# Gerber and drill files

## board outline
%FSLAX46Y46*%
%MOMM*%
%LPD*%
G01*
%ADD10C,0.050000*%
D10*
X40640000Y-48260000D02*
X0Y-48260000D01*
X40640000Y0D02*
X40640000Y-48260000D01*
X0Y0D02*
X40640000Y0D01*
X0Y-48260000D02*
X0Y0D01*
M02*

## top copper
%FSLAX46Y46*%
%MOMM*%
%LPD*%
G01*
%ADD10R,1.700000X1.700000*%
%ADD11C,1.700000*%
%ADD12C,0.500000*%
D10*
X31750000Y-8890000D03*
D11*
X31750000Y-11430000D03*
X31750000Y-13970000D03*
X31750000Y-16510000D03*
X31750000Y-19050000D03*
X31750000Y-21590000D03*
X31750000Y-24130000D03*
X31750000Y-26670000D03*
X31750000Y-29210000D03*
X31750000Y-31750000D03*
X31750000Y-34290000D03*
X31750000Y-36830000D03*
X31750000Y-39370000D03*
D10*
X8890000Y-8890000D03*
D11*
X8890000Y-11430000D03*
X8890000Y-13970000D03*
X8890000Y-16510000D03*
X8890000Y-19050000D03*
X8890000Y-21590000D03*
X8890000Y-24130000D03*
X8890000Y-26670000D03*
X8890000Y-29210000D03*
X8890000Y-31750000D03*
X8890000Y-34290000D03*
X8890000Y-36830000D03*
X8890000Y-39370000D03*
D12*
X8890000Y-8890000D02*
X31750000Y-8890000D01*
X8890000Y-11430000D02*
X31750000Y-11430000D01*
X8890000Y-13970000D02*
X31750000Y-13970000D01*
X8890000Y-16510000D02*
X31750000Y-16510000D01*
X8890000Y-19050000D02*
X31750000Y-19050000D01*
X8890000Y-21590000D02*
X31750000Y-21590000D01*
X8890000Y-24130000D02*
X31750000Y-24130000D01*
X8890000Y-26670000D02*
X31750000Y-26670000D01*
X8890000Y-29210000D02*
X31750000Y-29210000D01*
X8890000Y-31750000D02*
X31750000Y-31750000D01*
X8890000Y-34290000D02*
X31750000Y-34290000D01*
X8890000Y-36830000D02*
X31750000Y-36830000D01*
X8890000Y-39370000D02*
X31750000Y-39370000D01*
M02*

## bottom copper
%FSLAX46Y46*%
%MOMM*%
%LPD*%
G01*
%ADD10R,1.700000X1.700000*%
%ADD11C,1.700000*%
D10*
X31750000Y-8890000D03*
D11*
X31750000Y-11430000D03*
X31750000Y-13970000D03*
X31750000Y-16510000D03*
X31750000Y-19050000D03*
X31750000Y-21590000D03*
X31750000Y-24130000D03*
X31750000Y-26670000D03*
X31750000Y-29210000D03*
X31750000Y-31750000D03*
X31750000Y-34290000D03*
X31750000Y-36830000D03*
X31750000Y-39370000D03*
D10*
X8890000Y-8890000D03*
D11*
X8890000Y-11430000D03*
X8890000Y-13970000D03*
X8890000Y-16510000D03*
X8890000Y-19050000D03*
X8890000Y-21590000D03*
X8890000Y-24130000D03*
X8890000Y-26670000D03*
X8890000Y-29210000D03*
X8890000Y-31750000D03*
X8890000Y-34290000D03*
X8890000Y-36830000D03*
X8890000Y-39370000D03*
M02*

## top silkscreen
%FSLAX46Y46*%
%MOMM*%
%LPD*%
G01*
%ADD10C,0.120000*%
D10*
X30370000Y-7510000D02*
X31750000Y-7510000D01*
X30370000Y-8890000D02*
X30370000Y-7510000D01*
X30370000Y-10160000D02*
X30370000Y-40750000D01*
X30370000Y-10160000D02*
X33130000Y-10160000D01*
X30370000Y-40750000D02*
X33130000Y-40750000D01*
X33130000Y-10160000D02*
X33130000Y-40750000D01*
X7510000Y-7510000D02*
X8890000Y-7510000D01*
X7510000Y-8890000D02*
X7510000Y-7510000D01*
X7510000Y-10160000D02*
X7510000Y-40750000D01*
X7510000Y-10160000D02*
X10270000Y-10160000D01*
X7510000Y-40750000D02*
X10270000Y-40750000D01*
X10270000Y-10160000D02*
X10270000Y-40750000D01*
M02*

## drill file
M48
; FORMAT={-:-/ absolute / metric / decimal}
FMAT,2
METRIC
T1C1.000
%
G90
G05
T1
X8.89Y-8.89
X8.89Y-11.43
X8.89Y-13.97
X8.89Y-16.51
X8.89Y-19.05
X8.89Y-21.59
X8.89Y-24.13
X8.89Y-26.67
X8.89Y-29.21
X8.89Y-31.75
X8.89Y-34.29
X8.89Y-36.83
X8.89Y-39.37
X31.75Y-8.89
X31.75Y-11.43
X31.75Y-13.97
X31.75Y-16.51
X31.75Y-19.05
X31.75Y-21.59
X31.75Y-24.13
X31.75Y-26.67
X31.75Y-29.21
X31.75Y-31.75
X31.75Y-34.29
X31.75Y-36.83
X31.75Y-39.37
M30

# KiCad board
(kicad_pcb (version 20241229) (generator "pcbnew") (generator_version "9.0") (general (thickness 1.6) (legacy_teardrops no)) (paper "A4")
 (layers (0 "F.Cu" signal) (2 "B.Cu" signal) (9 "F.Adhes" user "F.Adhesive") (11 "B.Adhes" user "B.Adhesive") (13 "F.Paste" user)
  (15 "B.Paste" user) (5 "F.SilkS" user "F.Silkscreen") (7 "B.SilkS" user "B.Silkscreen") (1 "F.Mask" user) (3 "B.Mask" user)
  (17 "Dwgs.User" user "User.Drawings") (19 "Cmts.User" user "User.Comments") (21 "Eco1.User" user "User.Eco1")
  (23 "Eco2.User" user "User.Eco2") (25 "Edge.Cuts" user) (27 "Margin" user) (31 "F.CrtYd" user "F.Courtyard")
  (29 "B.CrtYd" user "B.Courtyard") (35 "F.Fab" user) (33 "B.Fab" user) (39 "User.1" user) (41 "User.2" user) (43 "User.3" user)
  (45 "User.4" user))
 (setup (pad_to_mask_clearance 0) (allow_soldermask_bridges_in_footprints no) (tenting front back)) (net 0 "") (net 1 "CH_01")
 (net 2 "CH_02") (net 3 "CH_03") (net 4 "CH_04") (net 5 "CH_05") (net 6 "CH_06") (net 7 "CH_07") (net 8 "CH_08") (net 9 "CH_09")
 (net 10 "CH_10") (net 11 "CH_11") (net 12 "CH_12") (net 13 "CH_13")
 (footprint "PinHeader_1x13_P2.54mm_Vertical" (layer "F.Cu") (at 31.75 8.89)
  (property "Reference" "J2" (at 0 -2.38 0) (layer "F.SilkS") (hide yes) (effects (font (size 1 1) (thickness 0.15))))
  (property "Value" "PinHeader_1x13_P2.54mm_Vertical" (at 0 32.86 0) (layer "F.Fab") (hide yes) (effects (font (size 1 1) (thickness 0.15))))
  (fp_line (start -1.38 -1.38) (end 0 -1.38) (stroke (width 0.12) (type solid)) (layer "F.SilkS"))
  (fp_line (start -1.38 0) (end -1.38 -1.38) (stroke (width 0.12) (type solid)) (layer "F.SilkS"))
  (fp_line (start -1.38 1.27) (end -1.38 31.86) (stroke (width 0.12) (type solid)) (layer "F.SilkS"))
  (fp_line (start -1.38 1.27) (end 1.38 1.27) (stroke (width 0.12) (type solid)) (layer "F.SilkS"))
  (fp_line (start -1.38 31.86) (end 1.38 31.86) (stroke (width 0.12) (type solid)) (layer "F.SilkS"))
  (fp_line (start 1.38 1.27) (end 1.38 31.86) (stroke (width 0.12) (type solid)) (layer "F.SilkS"))
  (pad "1" thru_hole rect (at 0 0) (size 1.7 1.7) (drill 1) (layers "*.Cu" "*.Mask") (remove_unused_layers no) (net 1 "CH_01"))
  (pad "2" thru_hole circle (at 0 2.54) (size 1.7 1.7) (drill 1) (layers "*.Cu" "*.Mask") (remove_unused_layers no) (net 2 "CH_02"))
  (pad "3" thru_hole circle (at 0 5.08) (size 1.7 1.7) (drill 1) (layers "*.Cu" "*.Mask") (remove_unused_layers no) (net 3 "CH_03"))
  (pad "4" thru_hole circle (at 0 7.62) (size 1.7 1.7) (drill 1) (layers "*.Cu" "*.Mask") (remove_unused_layers no) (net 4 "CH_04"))
  (pad "5" thru_hole circle (at 0 10.16) (size 1.7 1.7) (drill 1) (layers "*.Cu" "*.Mask") (remove_unused_layers no) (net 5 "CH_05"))
  (pad "6" thru_hole circle (at 0 12.7) (size 1.7 1.7) (drill 1) (layers "*.Cu" "*.Mask") (remove_unused_layers no) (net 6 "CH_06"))
  (pad "7" thru_hole circle (at 0 15.24) (size 1.7 1.7) (drill 1) (layers "*.Cu" "*.Mask") (remove_unused_layers no) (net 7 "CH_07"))
  (pad "8" thru_hole circle (at 0 17.78) (size 1.7 1.7) (drill 1) (layers "*.Cu" "*.Mask") (remove_unused_layers no) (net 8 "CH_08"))
  (pad "9" thru_hole circle (at 0 20.32) (size 1.7 1.7) (drill 1) (layers "*.Cu" "*.Mask") (remove_unused_layers no) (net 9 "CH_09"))
  (pad "10" thru_hole circle (at 0 22.86) (size 1.7 1.7) (drill 1) (layers "*.Cu" "*.Mask") (remove_unused_layers no) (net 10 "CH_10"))
  (pad "11" thru_hole circle (at 0 25.4) (size 1.7 1.7) (drill 1) (layers "*.Cu" "*.Mask") (remove_unused_layers no) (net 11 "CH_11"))
  (pad "12" thru_hole circle (at 0 27.94) (size 1.7 1.7) (drill 1) (layers "*.Cu" "*.Mask") (remove_unused_layers no) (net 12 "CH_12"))
  (pad "13" thru_hole circle (at 0 30.48) (size 1.7 1.7) (drill 1) (layers "*.Cu" "*.Mask") (remove_unused_layers no) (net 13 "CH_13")))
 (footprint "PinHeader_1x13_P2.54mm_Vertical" (layer "F.Cu") (at 8.89 8.89)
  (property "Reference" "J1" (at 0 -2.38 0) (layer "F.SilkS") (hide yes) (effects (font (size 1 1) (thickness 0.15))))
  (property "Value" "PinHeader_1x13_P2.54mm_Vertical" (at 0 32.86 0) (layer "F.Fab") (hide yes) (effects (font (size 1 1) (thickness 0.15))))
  (fp_line (start -1.38 -1.38) (end 0 -1.38) (stroke (width 0.12) (type solid)) (layer "F.SilkS"))
  (fp_line (start -1.38 0) (end -1.38 -1.38) (stroke (width 0.12) (type solid)) (layer "F.SilkS"))
  (fp_line (start -1.38 1.27) (end -1.38 31.86) (stroke (width 0.12) (type solid)) (layer "F.SilkS"))
  (fp_line (start -1.38 1.27) (end 1.38 1.27) (stroke (width 0.12) (type solid)) (layer "F.SilkS"))
  (fp_line (start -1.38 31.86) (end 1.38 31.86) (stroke (width 0.12) (type solid)) (layer "F.SilkS"))
  (fp_line (start 1.38 1.27) (end 1.38 31.86) (stroke (width 0.12) (type solid)) (layer "F.SilkS"))
  (pad "1" thru_hole rect (at 0 0) (size 1.7 1.7) (drill 1) (layers "*.Cu" "*.Mask") (remove_unused_layers no) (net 1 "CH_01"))
  (pad "2" thru_hole circle (at 0 2.54) (size 1.7 1.7) (drill 1) (layers "*.Cu" "*.Mask") (remove_unused_layers no) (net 2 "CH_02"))
  (pad "3" thru_hole circle (at 0 5.08) (size 1.7 1.7) (drill 1) (layers "*.Cu" "*.Mask") (remove_unused_layers no) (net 3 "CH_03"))
  (pad "4" thru_hole circle (at 0 7.62) (size 1.7 1.7) (drill 1) (layers "*.Cu" "*.Mask") (remove_unused_layers no) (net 4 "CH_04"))
  (pad "5" thru_hole circle (at 0 10.16) (size 1.7 1.7) (drill 1) (layers "*.Cu" "*.Mask") (remove_unused_layers no) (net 5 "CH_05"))
  (pad "6" thru_hole circle (at 0 12.7) (size 1.7 1.7) (drill 1) (layers "*.Cu" "*.Mask") (remove_unused_layers no) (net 6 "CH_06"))
  (pad "7" thru_hole circle (at 0 15.24) (size 1.7 1.7) (drill 1) (layers "*.Cu" "*.Mask") (remove_unused_layers no) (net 7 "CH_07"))
  (pad "8" thru_hole circle (at 0 17.78) (size 1.7 1.7) (drill 1) (layers "*.Cu" "*.Mask") (remove_unused_layers no) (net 8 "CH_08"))
  (pad "9" thru_hole circle (at 0 20.32) (size 1.7 1.7) (drill 1) (layers "*.Cu" "*.Mask") (remove_unused_layers no) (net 9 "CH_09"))
  (pad "10" thru_hole circle (at 0 22.86) (size 1.7 1.7) (drill 1) (layers "*.Cu" "*.Mask") (remove_unused_layers no) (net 10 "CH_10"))
  (pad "11" thru_hole circle (at 0 25.4) (size 1.7 1.7) (drill 1) (layers "*.Cu" "*.Mask") (remove_unused_layers no) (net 11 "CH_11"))
  (pad "12" thru_hole circle (at 0 27.94) (size 1.7 1.7) (drill 1) (layers "*.Cu" "*.Mask") (remove_unused_layers no) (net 12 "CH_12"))
  (pad "13" thru_hole circle (at 0 30.48) (size 1.7 1.7) (drill 1) (layers "*.Cu" "*.Mask") (remove_unused_layers no) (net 13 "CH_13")))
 (gr_line (start 40.64 48.26) (end 0 48.26) (stroke (width 0.05) (type default)) (layer "Edge.Cuts"))
 (gr_line (start 40.64 0) (end 40.64 48.26) (stroke (width 0.05) (type default)) (layer "Edge.Cuts"))
 (gr_line (start 0 0) (end 40.64 0) (stroke (width 0.05) (type default)) (layer "Edge.Cuts"))
 (gr_line (start 0 48.26) (end 0 0) (stroke (width 0.05) (type default)) (layer "Edge.Cuts"))
 (segment (start 8.89 8.89) (end 31.75 8.89) (width 0.5) (layer "F.Cu") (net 1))
 (segment (start 8.89 11.43) (end 31.75 11.43) (width 0.5) (layer "F.Cu") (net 2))
 (segment (start 8.89 13.97) (end 31.75 13.97) (width 0.5) (layer "F.Cu") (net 3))
 (segment (start 8.89 16.51) (end 31.75 16.51) (width 0.5) (layer "F.Cu") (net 4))
 (segment (start 8.89 19.05) (end 31.75 19.05) (width 0.5) (layer "F.Cu") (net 5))
 (segment (start 8.89 21.59) (end 31.75 21.59) (width 0.5) (layer "F.Cu") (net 6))
 (segment (start 8.89 24.13) (end 31.75 24.13) (width 0.5) (layer "F.Cu") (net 7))
 (segment (start 8.89 26.67) (end 31.75 26.67) (width 0.5) (layer "F.Cu") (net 8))
 (segment (start 8.89 29.21) (end 31.75 29.21) (width 0.5) (layer "F.Cu") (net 9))
 (segment (start 8.89 31.75) (end 31.75 31.75) (width 0.5) (layer "F.Cu") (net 10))
 (segment (start 8.89 34.29) (end 31.75 34.29) (width 0.5) (layer "F.Cu") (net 11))
 (segment (start 8.89 36.83) (end 31.75 36.83) (width 0.5) (layer "F.Cu") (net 12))
 (segment (start 8.89 39.37) (end 31.75 39.37) (width 0.5) (layer "F.Cu") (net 13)))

